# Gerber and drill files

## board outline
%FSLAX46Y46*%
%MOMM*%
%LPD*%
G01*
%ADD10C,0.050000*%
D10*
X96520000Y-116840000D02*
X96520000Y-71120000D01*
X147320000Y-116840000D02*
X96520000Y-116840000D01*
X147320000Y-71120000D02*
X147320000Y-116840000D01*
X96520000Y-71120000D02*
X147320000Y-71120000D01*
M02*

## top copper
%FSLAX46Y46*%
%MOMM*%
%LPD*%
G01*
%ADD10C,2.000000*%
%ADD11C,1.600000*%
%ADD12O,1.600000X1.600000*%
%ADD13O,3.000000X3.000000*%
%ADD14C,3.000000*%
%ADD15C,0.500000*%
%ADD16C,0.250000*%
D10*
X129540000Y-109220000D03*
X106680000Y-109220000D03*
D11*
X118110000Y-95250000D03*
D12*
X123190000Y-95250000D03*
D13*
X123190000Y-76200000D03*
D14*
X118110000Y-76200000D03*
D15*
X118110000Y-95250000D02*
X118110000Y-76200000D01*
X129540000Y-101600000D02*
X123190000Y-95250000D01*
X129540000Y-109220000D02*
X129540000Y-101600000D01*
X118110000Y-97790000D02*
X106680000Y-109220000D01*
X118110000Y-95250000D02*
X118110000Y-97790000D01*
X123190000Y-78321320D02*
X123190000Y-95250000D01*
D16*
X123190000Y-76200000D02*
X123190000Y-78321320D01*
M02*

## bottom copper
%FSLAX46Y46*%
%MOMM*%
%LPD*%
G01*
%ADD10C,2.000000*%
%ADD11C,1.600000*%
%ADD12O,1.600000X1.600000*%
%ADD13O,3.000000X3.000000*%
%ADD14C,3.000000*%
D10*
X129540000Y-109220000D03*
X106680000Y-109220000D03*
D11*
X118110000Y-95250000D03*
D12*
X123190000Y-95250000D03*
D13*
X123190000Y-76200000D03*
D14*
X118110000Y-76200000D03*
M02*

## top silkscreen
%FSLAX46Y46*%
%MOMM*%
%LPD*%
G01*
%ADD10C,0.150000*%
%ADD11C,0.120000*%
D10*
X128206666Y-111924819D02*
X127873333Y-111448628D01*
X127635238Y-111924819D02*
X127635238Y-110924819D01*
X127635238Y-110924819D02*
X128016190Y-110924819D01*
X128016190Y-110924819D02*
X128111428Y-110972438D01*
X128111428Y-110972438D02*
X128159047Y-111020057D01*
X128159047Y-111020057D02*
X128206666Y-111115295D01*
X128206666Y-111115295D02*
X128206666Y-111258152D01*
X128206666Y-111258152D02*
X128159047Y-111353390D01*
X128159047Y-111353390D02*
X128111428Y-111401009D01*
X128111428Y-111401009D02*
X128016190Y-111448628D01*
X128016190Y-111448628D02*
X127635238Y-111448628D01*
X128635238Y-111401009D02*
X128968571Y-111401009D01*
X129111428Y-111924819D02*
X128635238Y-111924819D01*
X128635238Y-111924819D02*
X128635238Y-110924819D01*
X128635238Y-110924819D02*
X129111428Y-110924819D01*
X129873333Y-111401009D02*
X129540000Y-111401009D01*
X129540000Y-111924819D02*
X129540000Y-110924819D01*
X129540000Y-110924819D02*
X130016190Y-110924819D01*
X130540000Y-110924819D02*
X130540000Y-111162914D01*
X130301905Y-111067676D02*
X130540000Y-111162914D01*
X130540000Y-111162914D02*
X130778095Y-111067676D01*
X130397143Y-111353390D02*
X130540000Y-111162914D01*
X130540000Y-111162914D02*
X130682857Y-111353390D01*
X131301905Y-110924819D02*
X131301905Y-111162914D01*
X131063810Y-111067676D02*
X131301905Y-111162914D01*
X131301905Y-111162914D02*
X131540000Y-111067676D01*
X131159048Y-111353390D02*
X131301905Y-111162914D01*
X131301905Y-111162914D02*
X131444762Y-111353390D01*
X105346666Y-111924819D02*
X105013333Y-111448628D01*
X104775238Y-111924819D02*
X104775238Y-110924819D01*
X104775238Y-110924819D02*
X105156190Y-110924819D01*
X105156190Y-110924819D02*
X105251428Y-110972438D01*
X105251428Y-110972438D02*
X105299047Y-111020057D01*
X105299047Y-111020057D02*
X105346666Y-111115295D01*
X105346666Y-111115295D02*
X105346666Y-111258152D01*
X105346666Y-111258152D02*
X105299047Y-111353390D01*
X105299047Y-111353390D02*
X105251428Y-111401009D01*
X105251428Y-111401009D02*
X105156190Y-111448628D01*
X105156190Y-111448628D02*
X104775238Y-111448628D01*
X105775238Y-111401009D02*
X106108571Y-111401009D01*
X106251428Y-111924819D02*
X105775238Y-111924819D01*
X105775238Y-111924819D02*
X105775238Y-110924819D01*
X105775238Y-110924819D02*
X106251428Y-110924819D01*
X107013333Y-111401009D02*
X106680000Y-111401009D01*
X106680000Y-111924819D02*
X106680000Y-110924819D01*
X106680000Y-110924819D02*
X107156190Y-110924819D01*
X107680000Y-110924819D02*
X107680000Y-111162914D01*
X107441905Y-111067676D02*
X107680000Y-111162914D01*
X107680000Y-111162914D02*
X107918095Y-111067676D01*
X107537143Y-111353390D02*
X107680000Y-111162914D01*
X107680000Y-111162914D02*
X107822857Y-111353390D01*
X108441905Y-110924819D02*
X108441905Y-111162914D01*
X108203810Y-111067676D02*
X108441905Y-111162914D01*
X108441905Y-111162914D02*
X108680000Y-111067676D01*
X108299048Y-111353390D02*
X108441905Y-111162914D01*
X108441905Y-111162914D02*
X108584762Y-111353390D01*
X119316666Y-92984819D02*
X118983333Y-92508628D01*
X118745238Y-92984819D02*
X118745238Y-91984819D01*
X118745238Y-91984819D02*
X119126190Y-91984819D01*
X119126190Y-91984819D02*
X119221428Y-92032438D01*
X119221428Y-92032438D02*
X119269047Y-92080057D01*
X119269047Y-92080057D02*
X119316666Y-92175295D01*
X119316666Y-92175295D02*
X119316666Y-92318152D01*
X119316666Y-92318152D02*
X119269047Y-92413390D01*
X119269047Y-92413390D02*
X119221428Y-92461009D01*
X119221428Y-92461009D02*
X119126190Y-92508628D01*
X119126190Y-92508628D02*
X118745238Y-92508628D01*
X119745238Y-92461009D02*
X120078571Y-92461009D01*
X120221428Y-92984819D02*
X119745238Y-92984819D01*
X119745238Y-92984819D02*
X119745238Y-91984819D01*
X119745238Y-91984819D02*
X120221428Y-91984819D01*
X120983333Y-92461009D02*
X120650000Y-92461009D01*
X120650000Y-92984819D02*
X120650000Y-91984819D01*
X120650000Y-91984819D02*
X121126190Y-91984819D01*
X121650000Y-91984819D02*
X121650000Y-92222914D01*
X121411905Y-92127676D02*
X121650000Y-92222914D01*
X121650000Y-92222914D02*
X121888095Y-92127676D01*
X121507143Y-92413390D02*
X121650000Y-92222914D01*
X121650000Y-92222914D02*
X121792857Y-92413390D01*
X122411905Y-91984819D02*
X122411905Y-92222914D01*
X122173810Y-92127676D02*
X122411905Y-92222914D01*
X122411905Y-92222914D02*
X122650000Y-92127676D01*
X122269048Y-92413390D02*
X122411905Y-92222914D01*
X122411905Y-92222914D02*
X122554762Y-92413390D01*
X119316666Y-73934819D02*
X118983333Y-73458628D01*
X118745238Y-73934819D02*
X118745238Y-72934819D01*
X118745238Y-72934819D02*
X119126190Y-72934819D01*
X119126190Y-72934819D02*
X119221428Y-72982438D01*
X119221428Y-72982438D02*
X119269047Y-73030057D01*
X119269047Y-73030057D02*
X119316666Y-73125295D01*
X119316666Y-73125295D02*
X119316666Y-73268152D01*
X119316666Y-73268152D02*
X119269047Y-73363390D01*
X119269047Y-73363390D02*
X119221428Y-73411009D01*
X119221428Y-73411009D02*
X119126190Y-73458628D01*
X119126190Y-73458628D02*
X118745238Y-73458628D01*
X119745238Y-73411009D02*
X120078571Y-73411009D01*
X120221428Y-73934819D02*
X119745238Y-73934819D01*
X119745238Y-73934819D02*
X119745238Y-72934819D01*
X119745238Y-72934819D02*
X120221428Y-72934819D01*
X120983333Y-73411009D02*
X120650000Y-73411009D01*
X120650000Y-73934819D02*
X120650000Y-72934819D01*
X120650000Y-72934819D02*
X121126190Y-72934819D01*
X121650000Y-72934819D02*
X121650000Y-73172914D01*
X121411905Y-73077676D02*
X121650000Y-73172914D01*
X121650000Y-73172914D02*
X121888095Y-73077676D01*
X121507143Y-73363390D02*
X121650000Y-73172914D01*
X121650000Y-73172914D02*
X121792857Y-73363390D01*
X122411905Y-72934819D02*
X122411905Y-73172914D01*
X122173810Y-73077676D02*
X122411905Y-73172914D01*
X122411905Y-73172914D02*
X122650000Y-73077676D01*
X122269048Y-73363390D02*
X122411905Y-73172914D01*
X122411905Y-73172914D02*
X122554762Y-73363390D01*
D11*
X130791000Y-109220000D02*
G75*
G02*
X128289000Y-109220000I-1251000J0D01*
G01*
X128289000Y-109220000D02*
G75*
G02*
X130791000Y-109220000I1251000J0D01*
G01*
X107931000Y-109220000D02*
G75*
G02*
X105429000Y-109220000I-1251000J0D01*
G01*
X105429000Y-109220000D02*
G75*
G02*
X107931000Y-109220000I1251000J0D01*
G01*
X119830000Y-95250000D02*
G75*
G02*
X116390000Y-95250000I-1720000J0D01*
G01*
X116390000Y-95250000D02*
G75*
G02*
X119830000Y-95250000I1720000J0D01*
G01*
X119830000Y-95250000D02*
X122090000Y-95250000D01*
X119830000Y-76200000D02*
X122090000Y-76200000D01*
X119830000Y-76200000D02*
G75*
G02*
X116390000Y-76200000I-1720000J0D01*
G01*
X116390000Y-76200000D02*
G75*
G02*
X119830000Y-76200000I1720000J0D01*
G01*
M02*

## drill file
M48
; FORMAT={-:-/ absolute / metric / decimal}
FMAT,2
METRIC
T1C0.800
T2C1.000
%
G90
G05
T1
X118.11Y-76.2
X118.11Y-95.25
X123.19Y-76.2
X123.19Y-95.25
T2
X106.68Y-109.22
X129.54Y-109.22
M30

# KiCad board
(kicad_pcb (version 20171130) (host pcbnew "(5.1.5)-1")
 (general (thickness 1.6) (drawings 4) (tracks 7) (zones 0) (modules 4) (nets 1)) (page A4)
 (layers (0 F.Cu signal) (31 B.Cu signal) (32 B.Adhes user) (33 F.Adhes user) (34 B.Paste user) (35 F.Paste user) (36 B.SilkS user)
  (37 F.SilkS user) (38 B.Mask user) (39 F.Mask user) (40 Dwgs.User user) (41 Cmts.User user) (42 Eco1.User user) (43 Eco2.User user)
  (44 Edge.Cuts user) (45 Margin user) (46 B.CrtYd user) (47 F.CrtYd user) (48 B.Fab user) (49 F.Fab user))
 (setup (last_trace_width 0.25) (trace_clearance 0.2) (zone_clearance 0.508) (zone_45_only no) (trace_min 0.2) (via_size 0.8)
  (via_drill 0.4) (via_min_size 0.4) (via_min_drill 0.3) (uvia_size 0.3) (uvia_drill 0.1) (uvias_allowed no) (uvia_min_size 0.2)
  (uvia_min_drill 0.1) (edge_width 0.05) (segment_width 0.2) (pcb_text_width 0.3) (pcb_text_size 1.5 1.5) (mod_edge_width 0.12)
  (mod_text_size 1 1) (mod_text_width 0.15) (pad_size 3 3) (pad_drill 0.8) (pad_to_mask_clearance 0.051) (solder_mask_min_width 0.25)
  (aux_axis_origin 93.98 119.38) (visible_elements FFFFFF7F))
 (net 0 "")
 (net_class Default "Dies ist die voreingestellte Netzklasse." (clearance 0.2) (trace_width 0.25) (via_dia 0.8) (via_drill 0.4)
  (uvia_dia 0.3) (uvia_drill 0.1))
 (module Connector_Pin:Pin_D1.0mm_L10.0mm (layer F.Cu) (at 129.54 109.22)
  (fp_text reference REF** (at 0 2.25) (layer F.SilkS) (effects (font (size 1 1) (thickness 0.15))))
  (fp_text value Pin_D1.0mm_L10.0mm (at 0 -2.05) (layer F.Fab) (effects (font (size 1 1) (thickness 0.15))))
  (fp_circle (center 0 0) (end 1.25 0.05) (layer F.SilkS) (width 0.12))
  (pad 1 thru_hole circle (at 0 0) (size 2 2) (drill 1) (layers *.Cu *.Mask)))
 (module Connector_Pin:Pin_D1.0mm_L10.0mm (layer F.Cu) (at 106.68 109.22)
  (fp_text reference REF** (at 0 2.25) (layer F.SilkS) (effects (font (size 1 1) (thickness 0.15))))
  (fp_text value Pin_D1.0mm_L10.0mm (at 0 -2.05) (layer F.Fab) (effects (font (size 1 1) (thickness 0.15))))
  (fp_circle (center 0 0) (end 1.25 0.05) (layer F.SilkS) (width 0.12))
  (pad 1 thru_hole circle (at 0 0) (size 2 2) (drill 1) (layers *.Cu *.Mask)))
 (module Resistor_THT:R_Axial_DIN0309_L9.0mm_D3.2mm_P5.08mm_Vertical (layer F.Cu) (at 118.11 95.25)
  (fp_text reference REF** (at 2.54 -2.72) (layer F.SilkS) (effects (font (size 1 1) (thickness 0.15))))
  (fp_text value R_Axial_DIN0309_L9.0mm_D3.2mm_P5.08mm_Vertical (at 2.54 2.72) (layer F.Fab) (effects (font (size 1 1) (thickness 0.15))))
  (fp_circle (center 0 0) (end 1.72 0) (layer F.SilkS) (width 0.12))
  (fp_line (start 1.72 0) (end 3.98 0) (layer F.SilkS) (width 0.12))
  (pad 1 thru_hole circle (at 0 0) (size 1.6 1.6) (drill 0.8) (layers *.Cu *.Mask))
  (pad 2 thru_hole oval (at 5.08 0) (size 1.6 1.6) (drill 0.8) (layers *.Cu *.Mask)))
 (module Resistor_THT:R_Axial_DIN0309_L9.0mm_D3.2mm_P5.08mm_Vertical (layer F.Cu) (at 118.11 76.2)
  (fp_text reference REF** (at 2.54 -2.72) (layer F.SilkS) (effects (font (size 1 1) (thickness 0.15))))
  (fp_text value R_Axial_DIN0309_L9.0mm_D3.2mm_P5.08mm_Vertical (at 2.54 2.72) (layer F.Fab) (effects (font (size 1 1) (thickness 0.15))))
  (fp_line (start 1.72 0) (end 3.98 0) (layer F.SilkS) (width 0.12))
  (fp_circle (center 0 0) (end 1.72 0) (layer F.SilkS) (width 0.12))
  (pad 2 thru_hole oval (at 5.08 0) (size 3 3) (drill 0.8) (layers *.Cu *.Mask))
  (pad 1 thru_hole circle (at 0 0) (size 3 3) (drill 0.8) (layers *.Cu *.Mask)))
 (gr_line (start 96.52 116.84) (end 96.52 71.12) (layer Edge.Cuts) (width 0.05))
 (gr_line (start 147.32 116.84) (end 96.52 116.84) (layer Edge.Cuts) (width 0.05))
 (gr_line (start 147.32 71.12) (end 147.32 116.84) (layer Edge.Cuts) (width 0.05))
 (gr_line (start 96.52 71.12) (end 147.32 71.12) (layer Edge.Cuts) (width 0.05))
 (segment (start 118.11 95.25) (end 118.11 76.2) (width 0.5) (layer F.Cu) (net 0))
 (segment (start 129.54 101.6) (end 123.19 95.25) (width 0.5) (layer F.Cu) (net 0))
 (segment (start 129.54 109.22) (end 129.54 101.6) (width 0.5) (layer F.Cu) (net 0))
 (segment (start 118.11 97.79) (end 106.68 109.22) (width 0.5) (layer F.Cu) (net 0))
 (segment (start 118.11 95.25) (end 118.11 97.79) (width 0.5) (layer F.Cu) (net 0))
 (segment (start 123.19 78.32132) (end 123.19 95.25) (width 0.5) (layer F.Cu) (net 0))
 (segment (start 123.19 76.2) (end 123.19 78.32132) (width 0.25) (layer F.Cu) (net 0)))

